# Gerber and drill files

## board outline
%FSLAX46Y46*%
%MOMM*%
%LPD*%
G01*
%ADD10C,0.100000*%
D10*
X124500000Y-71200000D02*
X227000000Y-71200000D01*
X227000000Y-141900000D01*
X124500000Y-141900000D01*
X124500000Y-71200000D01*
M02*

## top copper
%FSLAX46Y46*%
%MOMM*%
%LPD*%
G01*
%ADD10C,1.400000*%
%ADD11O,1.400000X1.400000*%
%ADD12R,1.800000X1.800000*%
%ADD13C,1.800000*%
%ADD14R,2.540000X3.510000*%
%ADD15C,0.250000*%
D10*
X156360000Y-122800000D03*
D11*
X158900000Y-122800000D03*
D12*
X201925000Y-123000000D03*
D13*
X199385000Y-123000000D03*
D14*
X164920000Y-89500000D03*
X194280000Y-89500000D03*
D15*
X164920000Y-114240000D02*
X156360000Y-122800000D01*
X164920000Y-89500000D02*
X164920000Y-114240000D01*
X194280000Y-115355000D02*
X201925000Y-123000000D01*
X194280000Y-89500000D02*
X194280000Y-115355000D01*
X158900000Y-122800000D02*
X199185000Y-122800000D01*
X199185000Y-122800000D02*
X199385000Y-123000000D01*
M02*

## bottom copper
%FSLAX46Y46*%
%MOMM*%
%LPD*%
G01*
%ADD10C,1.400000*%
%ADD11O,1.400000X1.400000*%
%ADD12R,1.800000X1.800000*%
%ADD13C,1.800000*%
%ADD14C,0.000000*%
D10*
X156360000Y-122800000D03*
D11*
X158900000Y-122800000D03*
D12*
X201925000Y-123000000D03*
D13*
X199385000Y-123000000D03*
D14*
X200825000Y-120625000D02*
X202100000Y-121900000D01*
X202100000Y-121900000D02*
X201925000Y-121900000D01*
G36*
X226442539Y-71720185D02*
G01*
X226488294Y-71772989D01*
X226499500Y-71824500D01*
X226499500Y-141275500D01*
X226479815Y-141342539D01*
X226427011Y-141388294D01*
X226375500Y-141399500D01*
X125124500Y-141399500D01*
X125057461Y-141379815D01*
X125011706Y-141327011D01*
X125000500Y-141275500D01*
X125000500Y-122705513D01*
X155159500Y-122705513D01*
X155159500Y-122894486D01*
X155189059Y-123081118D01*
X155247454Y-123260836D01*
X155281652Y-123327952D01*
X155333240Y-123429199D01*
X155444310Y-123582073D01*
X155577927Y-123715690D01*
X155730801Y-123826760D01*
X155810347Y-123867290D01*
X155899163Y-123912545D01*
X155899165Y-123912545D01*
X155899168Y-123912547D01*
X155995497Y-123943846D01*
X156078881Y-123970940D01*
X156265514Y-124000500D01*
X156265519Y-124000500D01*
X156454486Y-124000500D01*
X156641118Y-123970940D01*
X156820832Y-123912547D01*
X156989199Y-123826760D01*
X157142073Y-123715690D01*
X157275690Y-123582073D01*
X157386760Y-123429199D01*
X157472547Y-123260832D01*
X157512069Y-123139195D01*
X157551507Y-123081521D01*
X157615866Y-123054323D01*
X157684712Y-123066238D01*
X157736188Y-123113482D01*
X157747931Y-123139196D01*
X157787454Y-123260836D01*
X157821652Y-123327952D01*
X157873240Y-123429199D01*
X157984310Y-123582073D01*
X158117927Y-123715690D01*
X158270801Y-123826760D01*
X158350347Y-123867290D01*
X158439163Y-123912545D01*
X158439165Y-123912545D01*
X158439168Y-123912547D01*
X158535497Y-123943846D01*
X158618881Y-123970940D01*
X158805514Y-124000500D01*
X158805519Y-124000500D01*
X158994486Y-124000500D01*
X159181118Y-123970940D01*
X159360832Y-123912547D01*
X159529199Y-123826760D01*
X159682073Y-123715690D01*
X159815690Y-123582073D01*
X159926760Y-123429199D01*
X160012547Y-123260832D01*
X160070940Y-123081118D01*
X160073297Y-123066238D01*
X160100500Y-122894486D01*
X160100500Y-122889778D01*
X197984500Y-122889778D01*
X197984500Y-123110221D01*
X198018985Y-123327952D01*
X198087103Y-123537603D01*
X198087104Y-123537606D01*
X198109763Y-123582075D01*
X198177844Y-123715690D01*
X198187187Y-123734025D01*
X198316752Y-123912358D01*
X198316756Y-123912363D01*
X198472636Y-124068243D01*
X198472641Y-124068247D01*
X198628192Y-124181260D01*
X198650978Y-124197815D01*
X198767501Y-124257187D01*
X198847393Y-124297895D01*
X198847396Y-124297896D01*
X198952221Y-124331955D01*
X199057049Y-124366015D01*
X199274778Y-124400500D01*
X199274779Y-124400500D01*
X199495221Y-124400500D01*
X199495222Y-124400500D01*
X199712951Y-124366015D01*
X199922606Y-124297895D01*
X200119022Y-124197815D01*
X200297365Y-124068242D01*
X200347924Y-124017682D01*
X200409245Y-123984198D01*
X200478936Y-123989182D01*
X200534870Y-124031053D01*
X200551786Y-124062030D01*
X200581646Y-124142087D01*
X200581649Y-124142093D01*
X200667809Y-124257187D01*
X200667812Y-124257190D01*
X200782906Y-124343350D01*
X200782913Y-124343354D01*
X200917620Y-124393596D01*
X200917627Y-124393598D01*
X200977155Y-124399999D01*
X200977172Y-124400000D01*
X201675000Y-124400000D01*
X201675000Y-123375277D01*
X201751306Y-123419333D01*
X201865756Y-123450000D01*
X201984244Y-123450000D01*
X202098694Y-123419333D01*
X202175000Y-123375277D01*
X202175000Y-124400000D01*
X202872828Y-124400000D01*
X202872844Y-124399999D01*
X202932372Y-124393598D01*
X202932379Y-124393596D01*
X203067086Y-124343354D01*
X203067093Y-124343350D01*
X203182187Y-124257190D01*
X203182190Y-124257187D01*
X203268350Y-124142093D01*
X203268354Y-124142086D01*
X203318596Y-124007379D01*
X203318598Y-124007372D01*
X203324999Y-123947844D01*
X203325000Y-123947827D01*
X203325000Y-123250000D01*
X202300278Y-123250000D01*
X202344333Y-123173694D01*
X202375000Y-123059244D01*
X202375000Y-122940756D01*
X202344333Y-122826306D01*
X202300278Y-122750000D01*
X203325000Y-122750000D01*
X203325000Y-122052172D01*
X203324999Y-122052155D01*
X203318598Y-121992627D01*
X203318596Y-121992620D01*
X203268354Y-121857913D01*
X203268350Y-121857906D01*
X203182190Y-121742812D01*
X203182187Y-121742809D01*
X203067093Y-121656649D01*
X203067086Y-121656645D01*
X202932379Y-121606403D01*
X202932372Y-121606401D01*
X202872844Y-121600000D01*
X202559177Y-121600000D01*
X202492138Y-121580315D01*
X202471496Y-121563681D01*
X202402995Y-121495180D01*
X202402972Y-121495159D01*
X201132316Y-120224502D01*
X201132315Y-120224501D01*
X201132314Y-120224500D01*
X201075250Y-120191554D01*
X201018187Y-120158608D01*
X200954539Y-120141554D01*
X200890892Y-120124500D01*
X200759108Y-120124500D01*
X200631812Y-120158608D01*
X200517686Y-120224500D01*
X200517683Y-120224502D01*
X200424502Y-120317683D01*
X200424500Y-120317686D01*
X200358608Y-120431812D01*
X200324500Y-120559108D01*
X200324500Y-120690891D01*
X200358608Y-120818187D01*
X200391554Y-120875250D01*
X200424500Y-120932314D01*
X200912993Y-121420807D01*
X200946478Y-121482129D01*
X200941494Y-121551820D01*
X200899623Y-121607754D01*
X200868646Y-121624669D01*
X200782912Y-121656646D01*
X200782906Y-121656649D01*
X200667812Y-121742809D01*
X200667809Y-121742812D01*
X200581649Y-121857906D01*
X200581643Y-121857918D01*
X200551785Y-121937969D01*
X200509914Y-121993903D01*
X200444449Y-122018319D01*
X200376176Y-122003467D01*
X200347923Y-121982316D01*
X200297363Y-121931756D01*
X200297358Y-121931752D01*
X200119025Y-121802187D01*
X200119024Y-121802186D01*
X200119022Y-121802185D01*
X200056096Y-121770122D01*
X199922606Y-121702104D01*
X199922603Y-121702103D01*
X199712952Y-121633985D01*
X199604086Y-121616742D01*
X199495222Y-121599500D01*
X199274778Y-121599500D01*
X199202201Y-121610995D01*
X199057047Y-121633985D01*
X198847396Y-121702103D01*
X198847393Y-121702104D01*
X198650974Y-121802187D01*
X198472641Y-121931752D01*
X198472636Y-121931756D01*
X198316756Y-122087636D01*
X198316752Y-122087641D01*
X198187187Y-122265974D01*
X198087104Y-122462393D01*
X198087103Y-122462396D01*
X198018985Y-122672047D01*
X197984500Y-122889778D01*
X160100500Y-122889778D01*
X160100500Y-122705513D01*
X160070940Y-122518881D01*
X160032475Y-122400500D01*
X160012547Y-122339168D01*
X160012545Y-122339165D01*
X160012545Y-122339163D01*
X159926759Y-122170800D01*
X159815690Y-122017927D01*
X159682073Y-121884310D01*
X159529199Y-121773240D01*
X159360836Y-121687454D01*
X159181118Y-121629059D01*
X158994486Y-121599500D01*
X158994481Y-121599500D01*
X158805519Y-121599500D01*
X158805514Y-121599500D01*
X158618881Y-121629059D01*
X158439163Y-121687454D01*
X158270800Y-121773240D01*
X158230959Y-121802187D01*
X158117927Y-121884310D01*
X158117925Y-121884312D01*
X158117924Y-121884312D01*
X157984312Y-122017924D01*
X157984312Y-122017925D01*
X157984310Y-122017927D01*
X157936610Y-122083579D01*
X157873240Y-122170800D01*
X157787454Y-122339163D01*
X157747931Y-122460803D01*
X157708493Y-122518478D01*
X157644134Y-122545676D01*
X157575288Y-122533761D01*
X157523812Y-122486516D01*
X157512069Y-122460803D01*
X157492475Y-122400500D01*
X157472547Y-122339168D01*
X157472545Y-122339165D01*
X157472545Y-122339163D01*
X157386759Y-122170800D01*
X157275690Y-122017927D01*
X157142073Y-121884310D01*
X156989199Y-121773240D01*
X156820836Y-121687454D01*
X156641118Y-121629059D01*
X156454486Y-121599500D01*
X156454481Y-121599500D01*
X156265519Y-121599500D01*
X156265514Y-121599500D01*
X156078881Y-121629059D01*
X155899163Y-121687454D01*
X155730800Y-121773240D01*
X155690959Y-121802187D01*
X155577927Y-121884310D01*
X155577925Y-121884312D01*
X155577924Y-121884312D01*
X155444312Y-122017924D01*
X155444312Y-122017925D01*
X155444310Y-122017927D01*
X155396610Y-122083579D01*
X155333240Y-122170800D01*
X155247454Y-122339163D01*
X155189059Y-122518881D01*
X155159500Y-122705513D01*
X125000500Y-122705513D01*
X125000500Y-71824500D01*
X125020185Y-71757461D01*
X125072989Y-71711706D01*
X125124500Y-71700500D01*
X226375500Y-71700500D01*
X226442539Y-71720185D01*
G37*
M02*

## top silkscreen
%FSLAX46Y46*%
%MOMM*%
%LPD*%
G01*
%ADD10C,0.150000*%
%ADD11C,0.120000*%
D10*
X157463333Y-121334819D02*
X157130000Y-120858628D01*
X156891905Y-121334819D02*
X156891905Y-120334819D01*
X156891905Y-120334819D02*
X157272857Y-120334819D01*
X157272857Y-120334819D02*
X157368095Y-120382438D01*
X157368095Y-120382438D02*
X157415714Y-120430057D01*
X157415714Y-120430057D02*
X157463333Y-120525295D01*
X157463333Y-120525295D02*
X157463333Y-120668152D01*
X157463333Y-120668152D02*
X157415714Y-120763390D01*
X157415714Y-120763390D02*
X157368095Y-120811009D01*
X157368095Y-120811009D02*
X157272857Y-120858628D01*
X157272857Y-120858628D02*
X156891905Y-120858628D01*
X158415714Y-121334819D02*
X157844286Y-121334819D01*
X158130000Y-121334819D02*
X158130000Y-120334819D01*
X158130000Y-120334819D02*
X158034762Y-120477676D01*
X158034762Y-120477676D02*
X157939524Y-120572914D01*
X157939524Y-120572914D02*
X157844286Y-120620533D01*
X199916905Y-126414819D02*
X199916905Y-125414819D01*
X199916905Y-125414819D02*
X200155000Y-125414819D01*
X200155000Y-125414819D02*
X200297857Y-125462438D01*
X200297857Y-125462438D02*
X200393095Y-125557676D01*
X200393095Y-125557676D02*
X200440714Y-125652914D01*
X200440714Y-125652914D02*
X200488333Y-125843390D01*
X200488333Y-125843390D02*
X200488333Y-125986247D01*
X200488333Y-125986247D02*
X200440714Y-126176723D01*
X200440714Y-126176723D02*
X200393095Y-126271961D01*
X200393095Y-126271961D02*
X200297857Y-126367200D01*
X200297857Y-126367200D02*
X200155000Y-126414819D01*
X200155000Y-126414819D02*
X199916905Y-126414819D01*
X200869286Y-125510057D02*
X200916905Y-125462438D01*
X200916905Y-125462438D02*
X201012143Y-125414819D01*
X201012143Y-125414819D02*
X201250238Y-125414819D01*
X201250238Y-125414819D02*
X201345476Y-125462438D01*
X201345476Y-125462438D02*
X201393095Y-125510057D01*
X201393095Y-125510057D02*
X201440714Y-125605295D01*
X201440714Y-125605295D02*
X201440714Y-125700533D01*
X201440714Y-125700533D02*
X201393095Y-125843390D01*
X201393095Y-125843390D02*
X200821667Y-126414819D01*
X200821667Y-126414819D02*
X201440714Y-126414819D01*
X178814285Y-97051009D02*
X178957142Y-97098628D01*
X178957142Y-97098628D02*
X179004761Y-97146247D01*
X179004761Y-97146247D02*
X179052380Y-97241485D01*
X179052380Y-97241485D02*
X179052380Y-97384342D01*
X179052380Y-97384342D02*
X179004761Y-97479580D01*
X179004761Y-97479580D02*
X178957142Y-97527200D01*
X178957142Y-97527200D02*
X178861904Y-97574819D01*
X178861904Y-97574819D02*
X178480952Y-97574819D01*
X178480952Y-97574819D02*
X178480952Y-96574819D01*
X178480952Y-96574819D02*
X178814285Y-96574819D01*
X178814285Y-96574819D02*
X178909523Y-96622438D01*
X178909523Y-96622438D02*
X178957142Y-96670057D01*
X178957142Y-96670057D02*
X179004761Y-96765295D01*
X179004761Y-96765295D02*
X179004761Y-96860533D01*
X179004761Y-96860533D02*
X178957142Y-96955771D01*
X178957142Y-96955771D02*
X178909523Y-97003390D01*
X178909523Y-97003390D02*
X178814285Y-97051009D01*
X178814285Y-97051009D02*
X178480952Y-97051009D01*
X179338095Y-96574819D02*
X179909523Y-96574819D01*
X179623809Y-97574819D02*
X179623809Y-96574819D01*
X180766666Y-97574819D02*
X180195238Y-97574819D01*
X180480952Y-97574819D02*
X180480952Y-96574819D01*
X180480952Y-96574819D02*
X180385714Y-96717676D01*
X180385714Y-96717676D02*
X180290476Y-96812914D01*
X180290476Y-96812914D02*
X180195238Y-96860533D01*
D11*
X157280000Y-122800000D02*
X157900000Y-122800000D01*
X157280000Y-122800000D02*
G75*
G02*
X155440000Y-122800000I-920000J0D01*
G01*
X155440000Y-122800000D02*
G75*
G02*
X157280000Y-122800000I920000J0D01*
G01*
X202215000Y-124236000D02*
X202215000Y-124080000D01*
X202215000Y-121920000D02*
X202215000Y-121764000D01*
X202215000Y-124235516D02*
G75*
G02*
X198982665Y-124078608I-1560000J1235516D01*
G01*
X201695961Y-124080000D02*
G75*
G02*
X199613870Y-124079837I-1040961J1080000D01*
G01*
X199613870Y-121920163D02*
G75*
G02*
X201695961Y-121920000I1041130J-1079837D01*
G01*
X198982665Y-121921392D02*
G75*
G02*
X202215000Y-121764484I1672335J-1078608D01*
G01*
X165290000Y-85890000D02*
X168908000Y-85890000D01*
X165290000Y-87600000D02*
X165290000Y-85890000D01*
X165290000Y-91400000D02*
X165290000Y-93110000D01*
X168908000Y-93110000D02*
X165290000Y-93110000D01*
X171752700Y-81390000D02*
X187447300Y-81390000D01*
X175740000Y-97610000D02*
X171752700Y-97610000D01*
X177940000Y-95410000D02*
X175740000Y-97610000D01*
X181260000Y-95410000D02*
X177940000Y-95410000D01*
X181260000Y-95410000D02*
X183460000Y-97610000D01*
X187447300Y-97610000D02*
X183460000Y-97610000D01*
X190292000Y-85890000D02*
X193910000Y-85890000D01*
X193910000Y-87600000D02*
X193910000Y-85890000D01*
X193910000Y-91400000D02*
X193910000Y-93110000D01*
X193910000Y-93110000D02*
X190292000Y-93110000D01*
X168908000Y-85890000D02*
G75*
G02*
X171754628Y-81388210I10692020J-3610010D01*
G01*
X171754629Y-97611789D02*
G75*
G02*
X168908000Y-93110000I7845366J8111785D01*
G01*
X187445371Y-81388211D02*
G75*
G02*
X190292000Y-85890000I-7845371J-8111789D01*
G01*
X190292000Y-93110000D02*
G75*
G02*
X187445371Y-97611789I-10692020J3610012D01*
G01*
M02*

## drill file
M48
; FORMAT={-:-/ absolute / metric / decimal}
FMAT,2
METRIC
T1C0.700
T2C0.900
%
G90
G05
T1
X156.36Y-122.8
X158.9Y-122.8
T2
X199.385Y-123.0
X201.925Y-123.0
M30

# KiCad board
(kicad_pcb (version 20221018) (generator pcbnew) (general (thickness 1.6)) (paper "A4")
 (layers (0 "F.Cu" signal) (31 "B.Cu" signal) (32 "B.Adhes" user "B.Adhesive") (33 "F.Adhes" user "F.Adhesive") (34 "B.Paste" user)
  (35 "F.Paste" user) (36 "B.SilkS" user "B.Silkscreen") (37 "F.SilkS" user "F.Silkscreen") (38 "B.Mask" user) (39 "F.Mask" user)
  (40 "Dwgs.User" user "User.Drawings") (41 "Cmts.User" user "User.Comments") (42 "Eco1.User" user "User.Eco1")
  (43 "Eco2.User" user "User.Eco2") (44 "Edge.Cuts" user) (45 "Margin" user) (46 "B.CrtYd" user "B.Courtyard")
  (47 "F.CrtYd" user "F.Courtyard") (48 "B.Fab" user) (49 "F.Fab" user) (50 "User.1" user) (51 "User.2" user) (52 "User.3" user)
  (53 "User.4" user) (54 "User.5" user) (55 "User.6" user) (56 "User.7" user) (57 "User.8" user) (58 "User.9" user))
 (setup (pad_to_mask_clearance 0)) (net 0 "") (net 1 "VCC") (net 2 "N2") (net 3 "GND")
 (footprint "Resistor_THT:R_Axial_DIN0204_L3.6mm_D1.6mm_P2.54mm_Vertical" (layer "F.Cu") (at 156.36 122.8)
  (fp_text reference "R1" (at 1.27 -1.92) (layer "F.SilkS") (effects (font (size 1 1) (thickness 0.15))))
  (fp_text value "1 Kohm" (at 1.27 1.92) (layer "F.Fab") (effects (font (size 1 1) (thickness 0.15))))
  (fp_line (start 0.92 0) (end 1.54 0) (stroke (width 0.12) (type solid)) (layer "F.SilkS"))
  (fp_circle (center 0 0) (end 0.92 0) (stroke (width 0.12) (type solid)) (fill none) (layer "F.SilkS"))
  (pad "1" thru_hole circle (at 0 0) (size 1.4 1.4) (drill 0.7) (layers "*.Cu" "*.Mask") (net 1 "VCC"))
  (pad "2" thru_hole oval (at 2.54 0) (size 1.4 1.4) (drill 0.7) (layers "*.Cu" "*.Mask") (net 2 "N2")))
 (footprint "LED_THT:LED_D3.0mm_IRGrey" (layer "F.Cu") (at 201.925 123 180)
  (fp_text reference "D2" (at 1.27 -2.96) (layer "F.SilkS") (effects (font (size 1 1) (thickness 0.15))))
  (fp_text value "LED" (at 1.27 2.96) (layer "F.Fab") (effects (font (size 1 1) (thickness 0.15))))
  (fp_line (start -0.29 -1.236) (end -0.29 -1.08) (stroke (width 0.12) (type solid)) (layer "F.SilkS"))
  (fp_line (start -0.29 1.08) (end -0.29 1.236) (stroke (width 0.12) (type solid)) (layer "F.SilkS"))
  (fp_arc (start -0.29 -1.235516) (mid 1.366487 -1.987659) (end 2.942335 -1.078608) (stroke (width 0.12) (type solid)) (layer "F.SilkS"))
  (fp_arc (start 0.229039 -1.08) (mid 1.270117 -1.5) (end 2.31113 -1.079837) (stroke (width 0.12) (type solid)) (layer "F.SilkS"))
  (fp_arc (start 2.31113 1.079837) (mid 1.270117 1.5) (end 0.229039 1.08) (stroke (width 0.12) (type solid)) (layer "F.SilkS"))
  (fp_arc (start 2.942335 1.078608) (mid 1.366487 1.987659) (end -0.29 1.235516) (stroke (width 0.12) (type solid)) (layer "F.SilkS"))
  (pad "1" thru_hole rect (at 0 0 180) (size 1.8 1.8) (drill 0.9) (layers "*.Cu" "*.Mask") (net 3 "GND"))
  (pad "2" thru_hole circle (at 2.54 0 180) (size 1.8 1.8) (drill 0.9) (layers "*.Cu" "*.Mask") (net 2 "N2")))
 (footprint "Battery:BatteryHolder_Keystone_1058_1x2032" (layer "F.Cu") (at 179.6 89.5)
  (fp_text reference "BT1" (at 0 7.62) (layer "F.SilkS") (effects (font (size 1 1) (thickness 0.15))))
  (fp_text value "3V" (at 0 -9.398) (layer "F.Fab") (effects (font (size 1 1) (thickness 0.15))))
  (fp_line (start -14.31 -3.61) (end -10.692 -3.61) (stroke (width 0.12) (type solid)) (layer "F.SilkS"))
  (fp_line (start -14.31 -1.9) (end -14.31 -3.61) (stroke (width 0.12) (type solid)) (layer "F.SilkS"))
  (fp_line (start -14.31 1.9) (end -14.31 3.61) (stroke (width 0.12) (type solid)) (layer "F.SilkS"))
  (fp_line (start -10.692 3.61) (end -14.31 3.61) (stroke (width 0.12) (type solid)) (layer "F.SilkS"))
  (fp_line (start -7.8473 -8.11) (end 7.8473 -8.11) (stroke (width 0.12) (type solid)) (layer "F.SilkS"))
  (fp_line (start -3.86 8.11) (end -7.8473 8.11) (stroke (width 0.12) (type solid)) (layer "F.SilkS"))
  (fp_line (start -1.66 5.91) (end -3.86 8.11) (stroke (width 0.12) (type solid)) (layer "F.SilkS"))
  (fp_line (start 1.66 5.91) (end -1.66 5.91) (stroke (width 0.12) (type solid)) (layer "F.SilkS"))
  (fp_line (start 1.66 5.91) (end 3.86 8.11) (stroke (width 0.12) (type solid)) (layer "F.SilkS"))
  (fp_line (start 7.8473 8.11) (end 3.86 8.11) (stroke (width 0.12) (type solid)) (layer "F.SilkS"))
  (fp_line (start 10.692 -3.61) (end 14.31 -3.61) (stroke (width 0.12) (type solid)) (layer "F.SilkS"))
  (fp_line (start 14.31 -1.9) (end 14.31 -3.61) (stroke (width 0.12) (type solid)) (layer "F.SilkS"))
  (fp_line (start 14.31 1.9) (end 14.31 3.61) (stroke (width 0.12) (type solid)) (layer "F.SilkS"))
  (fp_line (start 14.31 3.61) (end 10.692 3.61) (stroke (width 0.12) (type solid)) (layer "F.SilkS"))
  (fp_arc (start -10.692 -3.61) (mid -9.538084 -6.031244) (end -7.845371 -8.111789) (stroke (width 0.12) (type solid)) (layer "F.SilkS"))
  (fp_arc (start -7.845371 8.111789) (mid -9.538085 6.031244) (end -10.692 3.61) (stroke (width 0.12) (type solid)) (layer "F.SilkS"))
  (fp_arc (start 7.845371 -8.111789) (mid 9.538085 -6.031244) (end 10.692 -3.61) (stroke (width 0.12) (type solid)) (layer "F.SilkS"))
  (fp_arc (start 10.692 3.61) (mid 9.538084 6.031244) (end 7.845371 8.111789) (stroke (width 0.12) (type solid)) (layer "F.SilkS"))
  (pad "1" smd rect (at -14.68 0) (size 2.54 3.51) (layers "F.Cu" "F.Paste" "F.Mask") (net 1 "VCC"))
  (pad "2" smd rect (at 14.68 0) (size 2.54 3.51) (layers "F.Cu" "F.Paste" "F.Mask") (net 3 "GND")))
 (gr_rect (start 124.5 71.2) (end 227 141.9) (stroke (width 0.1) (type default)) (fill none) (layer "Edge.Cuts"))
 (segment (start 200.825 120.625) (end 202.1 121.9) (width 0) (layer "B.Cu") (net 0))
 (segment (start 202.1 121.9) (end 201.925 121.9) (width 0) (layer "B.Cu") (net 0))
 (segment (start 164.92 114.24) (end 156.36 122.8) (width 0.25) (layer "F.Cu") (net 1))
 (segment (start 164.92 89.5) (end 164.92 114.24) (width 0.25) (layer "F.Cu") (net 1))
 (segment (start 194.28 115.355) (end 201.925 123) (width 0.25) (layer "F.Cu") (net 3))
 (segment (start 194.28 89.5) (end 194.28 115.355) (width 0.25) (layer "F.Cu") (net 3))
 (segment (start 158.9 122.8) (end 199.185 122.8) (width 0.25) (layer "F.Cu") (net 2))
 (segment (start 199.185 122.8) (end 199.385 123) (width 0.25) (layer "F.Cu") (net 2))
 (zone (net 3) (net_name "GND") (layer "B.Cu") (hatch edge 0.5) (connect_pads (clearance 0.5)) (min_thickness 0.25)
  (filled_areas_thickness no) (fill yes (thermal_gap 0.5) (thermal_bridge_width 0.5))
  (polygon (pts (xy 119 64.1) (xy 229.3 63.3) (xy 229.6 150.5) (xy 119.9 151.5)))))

